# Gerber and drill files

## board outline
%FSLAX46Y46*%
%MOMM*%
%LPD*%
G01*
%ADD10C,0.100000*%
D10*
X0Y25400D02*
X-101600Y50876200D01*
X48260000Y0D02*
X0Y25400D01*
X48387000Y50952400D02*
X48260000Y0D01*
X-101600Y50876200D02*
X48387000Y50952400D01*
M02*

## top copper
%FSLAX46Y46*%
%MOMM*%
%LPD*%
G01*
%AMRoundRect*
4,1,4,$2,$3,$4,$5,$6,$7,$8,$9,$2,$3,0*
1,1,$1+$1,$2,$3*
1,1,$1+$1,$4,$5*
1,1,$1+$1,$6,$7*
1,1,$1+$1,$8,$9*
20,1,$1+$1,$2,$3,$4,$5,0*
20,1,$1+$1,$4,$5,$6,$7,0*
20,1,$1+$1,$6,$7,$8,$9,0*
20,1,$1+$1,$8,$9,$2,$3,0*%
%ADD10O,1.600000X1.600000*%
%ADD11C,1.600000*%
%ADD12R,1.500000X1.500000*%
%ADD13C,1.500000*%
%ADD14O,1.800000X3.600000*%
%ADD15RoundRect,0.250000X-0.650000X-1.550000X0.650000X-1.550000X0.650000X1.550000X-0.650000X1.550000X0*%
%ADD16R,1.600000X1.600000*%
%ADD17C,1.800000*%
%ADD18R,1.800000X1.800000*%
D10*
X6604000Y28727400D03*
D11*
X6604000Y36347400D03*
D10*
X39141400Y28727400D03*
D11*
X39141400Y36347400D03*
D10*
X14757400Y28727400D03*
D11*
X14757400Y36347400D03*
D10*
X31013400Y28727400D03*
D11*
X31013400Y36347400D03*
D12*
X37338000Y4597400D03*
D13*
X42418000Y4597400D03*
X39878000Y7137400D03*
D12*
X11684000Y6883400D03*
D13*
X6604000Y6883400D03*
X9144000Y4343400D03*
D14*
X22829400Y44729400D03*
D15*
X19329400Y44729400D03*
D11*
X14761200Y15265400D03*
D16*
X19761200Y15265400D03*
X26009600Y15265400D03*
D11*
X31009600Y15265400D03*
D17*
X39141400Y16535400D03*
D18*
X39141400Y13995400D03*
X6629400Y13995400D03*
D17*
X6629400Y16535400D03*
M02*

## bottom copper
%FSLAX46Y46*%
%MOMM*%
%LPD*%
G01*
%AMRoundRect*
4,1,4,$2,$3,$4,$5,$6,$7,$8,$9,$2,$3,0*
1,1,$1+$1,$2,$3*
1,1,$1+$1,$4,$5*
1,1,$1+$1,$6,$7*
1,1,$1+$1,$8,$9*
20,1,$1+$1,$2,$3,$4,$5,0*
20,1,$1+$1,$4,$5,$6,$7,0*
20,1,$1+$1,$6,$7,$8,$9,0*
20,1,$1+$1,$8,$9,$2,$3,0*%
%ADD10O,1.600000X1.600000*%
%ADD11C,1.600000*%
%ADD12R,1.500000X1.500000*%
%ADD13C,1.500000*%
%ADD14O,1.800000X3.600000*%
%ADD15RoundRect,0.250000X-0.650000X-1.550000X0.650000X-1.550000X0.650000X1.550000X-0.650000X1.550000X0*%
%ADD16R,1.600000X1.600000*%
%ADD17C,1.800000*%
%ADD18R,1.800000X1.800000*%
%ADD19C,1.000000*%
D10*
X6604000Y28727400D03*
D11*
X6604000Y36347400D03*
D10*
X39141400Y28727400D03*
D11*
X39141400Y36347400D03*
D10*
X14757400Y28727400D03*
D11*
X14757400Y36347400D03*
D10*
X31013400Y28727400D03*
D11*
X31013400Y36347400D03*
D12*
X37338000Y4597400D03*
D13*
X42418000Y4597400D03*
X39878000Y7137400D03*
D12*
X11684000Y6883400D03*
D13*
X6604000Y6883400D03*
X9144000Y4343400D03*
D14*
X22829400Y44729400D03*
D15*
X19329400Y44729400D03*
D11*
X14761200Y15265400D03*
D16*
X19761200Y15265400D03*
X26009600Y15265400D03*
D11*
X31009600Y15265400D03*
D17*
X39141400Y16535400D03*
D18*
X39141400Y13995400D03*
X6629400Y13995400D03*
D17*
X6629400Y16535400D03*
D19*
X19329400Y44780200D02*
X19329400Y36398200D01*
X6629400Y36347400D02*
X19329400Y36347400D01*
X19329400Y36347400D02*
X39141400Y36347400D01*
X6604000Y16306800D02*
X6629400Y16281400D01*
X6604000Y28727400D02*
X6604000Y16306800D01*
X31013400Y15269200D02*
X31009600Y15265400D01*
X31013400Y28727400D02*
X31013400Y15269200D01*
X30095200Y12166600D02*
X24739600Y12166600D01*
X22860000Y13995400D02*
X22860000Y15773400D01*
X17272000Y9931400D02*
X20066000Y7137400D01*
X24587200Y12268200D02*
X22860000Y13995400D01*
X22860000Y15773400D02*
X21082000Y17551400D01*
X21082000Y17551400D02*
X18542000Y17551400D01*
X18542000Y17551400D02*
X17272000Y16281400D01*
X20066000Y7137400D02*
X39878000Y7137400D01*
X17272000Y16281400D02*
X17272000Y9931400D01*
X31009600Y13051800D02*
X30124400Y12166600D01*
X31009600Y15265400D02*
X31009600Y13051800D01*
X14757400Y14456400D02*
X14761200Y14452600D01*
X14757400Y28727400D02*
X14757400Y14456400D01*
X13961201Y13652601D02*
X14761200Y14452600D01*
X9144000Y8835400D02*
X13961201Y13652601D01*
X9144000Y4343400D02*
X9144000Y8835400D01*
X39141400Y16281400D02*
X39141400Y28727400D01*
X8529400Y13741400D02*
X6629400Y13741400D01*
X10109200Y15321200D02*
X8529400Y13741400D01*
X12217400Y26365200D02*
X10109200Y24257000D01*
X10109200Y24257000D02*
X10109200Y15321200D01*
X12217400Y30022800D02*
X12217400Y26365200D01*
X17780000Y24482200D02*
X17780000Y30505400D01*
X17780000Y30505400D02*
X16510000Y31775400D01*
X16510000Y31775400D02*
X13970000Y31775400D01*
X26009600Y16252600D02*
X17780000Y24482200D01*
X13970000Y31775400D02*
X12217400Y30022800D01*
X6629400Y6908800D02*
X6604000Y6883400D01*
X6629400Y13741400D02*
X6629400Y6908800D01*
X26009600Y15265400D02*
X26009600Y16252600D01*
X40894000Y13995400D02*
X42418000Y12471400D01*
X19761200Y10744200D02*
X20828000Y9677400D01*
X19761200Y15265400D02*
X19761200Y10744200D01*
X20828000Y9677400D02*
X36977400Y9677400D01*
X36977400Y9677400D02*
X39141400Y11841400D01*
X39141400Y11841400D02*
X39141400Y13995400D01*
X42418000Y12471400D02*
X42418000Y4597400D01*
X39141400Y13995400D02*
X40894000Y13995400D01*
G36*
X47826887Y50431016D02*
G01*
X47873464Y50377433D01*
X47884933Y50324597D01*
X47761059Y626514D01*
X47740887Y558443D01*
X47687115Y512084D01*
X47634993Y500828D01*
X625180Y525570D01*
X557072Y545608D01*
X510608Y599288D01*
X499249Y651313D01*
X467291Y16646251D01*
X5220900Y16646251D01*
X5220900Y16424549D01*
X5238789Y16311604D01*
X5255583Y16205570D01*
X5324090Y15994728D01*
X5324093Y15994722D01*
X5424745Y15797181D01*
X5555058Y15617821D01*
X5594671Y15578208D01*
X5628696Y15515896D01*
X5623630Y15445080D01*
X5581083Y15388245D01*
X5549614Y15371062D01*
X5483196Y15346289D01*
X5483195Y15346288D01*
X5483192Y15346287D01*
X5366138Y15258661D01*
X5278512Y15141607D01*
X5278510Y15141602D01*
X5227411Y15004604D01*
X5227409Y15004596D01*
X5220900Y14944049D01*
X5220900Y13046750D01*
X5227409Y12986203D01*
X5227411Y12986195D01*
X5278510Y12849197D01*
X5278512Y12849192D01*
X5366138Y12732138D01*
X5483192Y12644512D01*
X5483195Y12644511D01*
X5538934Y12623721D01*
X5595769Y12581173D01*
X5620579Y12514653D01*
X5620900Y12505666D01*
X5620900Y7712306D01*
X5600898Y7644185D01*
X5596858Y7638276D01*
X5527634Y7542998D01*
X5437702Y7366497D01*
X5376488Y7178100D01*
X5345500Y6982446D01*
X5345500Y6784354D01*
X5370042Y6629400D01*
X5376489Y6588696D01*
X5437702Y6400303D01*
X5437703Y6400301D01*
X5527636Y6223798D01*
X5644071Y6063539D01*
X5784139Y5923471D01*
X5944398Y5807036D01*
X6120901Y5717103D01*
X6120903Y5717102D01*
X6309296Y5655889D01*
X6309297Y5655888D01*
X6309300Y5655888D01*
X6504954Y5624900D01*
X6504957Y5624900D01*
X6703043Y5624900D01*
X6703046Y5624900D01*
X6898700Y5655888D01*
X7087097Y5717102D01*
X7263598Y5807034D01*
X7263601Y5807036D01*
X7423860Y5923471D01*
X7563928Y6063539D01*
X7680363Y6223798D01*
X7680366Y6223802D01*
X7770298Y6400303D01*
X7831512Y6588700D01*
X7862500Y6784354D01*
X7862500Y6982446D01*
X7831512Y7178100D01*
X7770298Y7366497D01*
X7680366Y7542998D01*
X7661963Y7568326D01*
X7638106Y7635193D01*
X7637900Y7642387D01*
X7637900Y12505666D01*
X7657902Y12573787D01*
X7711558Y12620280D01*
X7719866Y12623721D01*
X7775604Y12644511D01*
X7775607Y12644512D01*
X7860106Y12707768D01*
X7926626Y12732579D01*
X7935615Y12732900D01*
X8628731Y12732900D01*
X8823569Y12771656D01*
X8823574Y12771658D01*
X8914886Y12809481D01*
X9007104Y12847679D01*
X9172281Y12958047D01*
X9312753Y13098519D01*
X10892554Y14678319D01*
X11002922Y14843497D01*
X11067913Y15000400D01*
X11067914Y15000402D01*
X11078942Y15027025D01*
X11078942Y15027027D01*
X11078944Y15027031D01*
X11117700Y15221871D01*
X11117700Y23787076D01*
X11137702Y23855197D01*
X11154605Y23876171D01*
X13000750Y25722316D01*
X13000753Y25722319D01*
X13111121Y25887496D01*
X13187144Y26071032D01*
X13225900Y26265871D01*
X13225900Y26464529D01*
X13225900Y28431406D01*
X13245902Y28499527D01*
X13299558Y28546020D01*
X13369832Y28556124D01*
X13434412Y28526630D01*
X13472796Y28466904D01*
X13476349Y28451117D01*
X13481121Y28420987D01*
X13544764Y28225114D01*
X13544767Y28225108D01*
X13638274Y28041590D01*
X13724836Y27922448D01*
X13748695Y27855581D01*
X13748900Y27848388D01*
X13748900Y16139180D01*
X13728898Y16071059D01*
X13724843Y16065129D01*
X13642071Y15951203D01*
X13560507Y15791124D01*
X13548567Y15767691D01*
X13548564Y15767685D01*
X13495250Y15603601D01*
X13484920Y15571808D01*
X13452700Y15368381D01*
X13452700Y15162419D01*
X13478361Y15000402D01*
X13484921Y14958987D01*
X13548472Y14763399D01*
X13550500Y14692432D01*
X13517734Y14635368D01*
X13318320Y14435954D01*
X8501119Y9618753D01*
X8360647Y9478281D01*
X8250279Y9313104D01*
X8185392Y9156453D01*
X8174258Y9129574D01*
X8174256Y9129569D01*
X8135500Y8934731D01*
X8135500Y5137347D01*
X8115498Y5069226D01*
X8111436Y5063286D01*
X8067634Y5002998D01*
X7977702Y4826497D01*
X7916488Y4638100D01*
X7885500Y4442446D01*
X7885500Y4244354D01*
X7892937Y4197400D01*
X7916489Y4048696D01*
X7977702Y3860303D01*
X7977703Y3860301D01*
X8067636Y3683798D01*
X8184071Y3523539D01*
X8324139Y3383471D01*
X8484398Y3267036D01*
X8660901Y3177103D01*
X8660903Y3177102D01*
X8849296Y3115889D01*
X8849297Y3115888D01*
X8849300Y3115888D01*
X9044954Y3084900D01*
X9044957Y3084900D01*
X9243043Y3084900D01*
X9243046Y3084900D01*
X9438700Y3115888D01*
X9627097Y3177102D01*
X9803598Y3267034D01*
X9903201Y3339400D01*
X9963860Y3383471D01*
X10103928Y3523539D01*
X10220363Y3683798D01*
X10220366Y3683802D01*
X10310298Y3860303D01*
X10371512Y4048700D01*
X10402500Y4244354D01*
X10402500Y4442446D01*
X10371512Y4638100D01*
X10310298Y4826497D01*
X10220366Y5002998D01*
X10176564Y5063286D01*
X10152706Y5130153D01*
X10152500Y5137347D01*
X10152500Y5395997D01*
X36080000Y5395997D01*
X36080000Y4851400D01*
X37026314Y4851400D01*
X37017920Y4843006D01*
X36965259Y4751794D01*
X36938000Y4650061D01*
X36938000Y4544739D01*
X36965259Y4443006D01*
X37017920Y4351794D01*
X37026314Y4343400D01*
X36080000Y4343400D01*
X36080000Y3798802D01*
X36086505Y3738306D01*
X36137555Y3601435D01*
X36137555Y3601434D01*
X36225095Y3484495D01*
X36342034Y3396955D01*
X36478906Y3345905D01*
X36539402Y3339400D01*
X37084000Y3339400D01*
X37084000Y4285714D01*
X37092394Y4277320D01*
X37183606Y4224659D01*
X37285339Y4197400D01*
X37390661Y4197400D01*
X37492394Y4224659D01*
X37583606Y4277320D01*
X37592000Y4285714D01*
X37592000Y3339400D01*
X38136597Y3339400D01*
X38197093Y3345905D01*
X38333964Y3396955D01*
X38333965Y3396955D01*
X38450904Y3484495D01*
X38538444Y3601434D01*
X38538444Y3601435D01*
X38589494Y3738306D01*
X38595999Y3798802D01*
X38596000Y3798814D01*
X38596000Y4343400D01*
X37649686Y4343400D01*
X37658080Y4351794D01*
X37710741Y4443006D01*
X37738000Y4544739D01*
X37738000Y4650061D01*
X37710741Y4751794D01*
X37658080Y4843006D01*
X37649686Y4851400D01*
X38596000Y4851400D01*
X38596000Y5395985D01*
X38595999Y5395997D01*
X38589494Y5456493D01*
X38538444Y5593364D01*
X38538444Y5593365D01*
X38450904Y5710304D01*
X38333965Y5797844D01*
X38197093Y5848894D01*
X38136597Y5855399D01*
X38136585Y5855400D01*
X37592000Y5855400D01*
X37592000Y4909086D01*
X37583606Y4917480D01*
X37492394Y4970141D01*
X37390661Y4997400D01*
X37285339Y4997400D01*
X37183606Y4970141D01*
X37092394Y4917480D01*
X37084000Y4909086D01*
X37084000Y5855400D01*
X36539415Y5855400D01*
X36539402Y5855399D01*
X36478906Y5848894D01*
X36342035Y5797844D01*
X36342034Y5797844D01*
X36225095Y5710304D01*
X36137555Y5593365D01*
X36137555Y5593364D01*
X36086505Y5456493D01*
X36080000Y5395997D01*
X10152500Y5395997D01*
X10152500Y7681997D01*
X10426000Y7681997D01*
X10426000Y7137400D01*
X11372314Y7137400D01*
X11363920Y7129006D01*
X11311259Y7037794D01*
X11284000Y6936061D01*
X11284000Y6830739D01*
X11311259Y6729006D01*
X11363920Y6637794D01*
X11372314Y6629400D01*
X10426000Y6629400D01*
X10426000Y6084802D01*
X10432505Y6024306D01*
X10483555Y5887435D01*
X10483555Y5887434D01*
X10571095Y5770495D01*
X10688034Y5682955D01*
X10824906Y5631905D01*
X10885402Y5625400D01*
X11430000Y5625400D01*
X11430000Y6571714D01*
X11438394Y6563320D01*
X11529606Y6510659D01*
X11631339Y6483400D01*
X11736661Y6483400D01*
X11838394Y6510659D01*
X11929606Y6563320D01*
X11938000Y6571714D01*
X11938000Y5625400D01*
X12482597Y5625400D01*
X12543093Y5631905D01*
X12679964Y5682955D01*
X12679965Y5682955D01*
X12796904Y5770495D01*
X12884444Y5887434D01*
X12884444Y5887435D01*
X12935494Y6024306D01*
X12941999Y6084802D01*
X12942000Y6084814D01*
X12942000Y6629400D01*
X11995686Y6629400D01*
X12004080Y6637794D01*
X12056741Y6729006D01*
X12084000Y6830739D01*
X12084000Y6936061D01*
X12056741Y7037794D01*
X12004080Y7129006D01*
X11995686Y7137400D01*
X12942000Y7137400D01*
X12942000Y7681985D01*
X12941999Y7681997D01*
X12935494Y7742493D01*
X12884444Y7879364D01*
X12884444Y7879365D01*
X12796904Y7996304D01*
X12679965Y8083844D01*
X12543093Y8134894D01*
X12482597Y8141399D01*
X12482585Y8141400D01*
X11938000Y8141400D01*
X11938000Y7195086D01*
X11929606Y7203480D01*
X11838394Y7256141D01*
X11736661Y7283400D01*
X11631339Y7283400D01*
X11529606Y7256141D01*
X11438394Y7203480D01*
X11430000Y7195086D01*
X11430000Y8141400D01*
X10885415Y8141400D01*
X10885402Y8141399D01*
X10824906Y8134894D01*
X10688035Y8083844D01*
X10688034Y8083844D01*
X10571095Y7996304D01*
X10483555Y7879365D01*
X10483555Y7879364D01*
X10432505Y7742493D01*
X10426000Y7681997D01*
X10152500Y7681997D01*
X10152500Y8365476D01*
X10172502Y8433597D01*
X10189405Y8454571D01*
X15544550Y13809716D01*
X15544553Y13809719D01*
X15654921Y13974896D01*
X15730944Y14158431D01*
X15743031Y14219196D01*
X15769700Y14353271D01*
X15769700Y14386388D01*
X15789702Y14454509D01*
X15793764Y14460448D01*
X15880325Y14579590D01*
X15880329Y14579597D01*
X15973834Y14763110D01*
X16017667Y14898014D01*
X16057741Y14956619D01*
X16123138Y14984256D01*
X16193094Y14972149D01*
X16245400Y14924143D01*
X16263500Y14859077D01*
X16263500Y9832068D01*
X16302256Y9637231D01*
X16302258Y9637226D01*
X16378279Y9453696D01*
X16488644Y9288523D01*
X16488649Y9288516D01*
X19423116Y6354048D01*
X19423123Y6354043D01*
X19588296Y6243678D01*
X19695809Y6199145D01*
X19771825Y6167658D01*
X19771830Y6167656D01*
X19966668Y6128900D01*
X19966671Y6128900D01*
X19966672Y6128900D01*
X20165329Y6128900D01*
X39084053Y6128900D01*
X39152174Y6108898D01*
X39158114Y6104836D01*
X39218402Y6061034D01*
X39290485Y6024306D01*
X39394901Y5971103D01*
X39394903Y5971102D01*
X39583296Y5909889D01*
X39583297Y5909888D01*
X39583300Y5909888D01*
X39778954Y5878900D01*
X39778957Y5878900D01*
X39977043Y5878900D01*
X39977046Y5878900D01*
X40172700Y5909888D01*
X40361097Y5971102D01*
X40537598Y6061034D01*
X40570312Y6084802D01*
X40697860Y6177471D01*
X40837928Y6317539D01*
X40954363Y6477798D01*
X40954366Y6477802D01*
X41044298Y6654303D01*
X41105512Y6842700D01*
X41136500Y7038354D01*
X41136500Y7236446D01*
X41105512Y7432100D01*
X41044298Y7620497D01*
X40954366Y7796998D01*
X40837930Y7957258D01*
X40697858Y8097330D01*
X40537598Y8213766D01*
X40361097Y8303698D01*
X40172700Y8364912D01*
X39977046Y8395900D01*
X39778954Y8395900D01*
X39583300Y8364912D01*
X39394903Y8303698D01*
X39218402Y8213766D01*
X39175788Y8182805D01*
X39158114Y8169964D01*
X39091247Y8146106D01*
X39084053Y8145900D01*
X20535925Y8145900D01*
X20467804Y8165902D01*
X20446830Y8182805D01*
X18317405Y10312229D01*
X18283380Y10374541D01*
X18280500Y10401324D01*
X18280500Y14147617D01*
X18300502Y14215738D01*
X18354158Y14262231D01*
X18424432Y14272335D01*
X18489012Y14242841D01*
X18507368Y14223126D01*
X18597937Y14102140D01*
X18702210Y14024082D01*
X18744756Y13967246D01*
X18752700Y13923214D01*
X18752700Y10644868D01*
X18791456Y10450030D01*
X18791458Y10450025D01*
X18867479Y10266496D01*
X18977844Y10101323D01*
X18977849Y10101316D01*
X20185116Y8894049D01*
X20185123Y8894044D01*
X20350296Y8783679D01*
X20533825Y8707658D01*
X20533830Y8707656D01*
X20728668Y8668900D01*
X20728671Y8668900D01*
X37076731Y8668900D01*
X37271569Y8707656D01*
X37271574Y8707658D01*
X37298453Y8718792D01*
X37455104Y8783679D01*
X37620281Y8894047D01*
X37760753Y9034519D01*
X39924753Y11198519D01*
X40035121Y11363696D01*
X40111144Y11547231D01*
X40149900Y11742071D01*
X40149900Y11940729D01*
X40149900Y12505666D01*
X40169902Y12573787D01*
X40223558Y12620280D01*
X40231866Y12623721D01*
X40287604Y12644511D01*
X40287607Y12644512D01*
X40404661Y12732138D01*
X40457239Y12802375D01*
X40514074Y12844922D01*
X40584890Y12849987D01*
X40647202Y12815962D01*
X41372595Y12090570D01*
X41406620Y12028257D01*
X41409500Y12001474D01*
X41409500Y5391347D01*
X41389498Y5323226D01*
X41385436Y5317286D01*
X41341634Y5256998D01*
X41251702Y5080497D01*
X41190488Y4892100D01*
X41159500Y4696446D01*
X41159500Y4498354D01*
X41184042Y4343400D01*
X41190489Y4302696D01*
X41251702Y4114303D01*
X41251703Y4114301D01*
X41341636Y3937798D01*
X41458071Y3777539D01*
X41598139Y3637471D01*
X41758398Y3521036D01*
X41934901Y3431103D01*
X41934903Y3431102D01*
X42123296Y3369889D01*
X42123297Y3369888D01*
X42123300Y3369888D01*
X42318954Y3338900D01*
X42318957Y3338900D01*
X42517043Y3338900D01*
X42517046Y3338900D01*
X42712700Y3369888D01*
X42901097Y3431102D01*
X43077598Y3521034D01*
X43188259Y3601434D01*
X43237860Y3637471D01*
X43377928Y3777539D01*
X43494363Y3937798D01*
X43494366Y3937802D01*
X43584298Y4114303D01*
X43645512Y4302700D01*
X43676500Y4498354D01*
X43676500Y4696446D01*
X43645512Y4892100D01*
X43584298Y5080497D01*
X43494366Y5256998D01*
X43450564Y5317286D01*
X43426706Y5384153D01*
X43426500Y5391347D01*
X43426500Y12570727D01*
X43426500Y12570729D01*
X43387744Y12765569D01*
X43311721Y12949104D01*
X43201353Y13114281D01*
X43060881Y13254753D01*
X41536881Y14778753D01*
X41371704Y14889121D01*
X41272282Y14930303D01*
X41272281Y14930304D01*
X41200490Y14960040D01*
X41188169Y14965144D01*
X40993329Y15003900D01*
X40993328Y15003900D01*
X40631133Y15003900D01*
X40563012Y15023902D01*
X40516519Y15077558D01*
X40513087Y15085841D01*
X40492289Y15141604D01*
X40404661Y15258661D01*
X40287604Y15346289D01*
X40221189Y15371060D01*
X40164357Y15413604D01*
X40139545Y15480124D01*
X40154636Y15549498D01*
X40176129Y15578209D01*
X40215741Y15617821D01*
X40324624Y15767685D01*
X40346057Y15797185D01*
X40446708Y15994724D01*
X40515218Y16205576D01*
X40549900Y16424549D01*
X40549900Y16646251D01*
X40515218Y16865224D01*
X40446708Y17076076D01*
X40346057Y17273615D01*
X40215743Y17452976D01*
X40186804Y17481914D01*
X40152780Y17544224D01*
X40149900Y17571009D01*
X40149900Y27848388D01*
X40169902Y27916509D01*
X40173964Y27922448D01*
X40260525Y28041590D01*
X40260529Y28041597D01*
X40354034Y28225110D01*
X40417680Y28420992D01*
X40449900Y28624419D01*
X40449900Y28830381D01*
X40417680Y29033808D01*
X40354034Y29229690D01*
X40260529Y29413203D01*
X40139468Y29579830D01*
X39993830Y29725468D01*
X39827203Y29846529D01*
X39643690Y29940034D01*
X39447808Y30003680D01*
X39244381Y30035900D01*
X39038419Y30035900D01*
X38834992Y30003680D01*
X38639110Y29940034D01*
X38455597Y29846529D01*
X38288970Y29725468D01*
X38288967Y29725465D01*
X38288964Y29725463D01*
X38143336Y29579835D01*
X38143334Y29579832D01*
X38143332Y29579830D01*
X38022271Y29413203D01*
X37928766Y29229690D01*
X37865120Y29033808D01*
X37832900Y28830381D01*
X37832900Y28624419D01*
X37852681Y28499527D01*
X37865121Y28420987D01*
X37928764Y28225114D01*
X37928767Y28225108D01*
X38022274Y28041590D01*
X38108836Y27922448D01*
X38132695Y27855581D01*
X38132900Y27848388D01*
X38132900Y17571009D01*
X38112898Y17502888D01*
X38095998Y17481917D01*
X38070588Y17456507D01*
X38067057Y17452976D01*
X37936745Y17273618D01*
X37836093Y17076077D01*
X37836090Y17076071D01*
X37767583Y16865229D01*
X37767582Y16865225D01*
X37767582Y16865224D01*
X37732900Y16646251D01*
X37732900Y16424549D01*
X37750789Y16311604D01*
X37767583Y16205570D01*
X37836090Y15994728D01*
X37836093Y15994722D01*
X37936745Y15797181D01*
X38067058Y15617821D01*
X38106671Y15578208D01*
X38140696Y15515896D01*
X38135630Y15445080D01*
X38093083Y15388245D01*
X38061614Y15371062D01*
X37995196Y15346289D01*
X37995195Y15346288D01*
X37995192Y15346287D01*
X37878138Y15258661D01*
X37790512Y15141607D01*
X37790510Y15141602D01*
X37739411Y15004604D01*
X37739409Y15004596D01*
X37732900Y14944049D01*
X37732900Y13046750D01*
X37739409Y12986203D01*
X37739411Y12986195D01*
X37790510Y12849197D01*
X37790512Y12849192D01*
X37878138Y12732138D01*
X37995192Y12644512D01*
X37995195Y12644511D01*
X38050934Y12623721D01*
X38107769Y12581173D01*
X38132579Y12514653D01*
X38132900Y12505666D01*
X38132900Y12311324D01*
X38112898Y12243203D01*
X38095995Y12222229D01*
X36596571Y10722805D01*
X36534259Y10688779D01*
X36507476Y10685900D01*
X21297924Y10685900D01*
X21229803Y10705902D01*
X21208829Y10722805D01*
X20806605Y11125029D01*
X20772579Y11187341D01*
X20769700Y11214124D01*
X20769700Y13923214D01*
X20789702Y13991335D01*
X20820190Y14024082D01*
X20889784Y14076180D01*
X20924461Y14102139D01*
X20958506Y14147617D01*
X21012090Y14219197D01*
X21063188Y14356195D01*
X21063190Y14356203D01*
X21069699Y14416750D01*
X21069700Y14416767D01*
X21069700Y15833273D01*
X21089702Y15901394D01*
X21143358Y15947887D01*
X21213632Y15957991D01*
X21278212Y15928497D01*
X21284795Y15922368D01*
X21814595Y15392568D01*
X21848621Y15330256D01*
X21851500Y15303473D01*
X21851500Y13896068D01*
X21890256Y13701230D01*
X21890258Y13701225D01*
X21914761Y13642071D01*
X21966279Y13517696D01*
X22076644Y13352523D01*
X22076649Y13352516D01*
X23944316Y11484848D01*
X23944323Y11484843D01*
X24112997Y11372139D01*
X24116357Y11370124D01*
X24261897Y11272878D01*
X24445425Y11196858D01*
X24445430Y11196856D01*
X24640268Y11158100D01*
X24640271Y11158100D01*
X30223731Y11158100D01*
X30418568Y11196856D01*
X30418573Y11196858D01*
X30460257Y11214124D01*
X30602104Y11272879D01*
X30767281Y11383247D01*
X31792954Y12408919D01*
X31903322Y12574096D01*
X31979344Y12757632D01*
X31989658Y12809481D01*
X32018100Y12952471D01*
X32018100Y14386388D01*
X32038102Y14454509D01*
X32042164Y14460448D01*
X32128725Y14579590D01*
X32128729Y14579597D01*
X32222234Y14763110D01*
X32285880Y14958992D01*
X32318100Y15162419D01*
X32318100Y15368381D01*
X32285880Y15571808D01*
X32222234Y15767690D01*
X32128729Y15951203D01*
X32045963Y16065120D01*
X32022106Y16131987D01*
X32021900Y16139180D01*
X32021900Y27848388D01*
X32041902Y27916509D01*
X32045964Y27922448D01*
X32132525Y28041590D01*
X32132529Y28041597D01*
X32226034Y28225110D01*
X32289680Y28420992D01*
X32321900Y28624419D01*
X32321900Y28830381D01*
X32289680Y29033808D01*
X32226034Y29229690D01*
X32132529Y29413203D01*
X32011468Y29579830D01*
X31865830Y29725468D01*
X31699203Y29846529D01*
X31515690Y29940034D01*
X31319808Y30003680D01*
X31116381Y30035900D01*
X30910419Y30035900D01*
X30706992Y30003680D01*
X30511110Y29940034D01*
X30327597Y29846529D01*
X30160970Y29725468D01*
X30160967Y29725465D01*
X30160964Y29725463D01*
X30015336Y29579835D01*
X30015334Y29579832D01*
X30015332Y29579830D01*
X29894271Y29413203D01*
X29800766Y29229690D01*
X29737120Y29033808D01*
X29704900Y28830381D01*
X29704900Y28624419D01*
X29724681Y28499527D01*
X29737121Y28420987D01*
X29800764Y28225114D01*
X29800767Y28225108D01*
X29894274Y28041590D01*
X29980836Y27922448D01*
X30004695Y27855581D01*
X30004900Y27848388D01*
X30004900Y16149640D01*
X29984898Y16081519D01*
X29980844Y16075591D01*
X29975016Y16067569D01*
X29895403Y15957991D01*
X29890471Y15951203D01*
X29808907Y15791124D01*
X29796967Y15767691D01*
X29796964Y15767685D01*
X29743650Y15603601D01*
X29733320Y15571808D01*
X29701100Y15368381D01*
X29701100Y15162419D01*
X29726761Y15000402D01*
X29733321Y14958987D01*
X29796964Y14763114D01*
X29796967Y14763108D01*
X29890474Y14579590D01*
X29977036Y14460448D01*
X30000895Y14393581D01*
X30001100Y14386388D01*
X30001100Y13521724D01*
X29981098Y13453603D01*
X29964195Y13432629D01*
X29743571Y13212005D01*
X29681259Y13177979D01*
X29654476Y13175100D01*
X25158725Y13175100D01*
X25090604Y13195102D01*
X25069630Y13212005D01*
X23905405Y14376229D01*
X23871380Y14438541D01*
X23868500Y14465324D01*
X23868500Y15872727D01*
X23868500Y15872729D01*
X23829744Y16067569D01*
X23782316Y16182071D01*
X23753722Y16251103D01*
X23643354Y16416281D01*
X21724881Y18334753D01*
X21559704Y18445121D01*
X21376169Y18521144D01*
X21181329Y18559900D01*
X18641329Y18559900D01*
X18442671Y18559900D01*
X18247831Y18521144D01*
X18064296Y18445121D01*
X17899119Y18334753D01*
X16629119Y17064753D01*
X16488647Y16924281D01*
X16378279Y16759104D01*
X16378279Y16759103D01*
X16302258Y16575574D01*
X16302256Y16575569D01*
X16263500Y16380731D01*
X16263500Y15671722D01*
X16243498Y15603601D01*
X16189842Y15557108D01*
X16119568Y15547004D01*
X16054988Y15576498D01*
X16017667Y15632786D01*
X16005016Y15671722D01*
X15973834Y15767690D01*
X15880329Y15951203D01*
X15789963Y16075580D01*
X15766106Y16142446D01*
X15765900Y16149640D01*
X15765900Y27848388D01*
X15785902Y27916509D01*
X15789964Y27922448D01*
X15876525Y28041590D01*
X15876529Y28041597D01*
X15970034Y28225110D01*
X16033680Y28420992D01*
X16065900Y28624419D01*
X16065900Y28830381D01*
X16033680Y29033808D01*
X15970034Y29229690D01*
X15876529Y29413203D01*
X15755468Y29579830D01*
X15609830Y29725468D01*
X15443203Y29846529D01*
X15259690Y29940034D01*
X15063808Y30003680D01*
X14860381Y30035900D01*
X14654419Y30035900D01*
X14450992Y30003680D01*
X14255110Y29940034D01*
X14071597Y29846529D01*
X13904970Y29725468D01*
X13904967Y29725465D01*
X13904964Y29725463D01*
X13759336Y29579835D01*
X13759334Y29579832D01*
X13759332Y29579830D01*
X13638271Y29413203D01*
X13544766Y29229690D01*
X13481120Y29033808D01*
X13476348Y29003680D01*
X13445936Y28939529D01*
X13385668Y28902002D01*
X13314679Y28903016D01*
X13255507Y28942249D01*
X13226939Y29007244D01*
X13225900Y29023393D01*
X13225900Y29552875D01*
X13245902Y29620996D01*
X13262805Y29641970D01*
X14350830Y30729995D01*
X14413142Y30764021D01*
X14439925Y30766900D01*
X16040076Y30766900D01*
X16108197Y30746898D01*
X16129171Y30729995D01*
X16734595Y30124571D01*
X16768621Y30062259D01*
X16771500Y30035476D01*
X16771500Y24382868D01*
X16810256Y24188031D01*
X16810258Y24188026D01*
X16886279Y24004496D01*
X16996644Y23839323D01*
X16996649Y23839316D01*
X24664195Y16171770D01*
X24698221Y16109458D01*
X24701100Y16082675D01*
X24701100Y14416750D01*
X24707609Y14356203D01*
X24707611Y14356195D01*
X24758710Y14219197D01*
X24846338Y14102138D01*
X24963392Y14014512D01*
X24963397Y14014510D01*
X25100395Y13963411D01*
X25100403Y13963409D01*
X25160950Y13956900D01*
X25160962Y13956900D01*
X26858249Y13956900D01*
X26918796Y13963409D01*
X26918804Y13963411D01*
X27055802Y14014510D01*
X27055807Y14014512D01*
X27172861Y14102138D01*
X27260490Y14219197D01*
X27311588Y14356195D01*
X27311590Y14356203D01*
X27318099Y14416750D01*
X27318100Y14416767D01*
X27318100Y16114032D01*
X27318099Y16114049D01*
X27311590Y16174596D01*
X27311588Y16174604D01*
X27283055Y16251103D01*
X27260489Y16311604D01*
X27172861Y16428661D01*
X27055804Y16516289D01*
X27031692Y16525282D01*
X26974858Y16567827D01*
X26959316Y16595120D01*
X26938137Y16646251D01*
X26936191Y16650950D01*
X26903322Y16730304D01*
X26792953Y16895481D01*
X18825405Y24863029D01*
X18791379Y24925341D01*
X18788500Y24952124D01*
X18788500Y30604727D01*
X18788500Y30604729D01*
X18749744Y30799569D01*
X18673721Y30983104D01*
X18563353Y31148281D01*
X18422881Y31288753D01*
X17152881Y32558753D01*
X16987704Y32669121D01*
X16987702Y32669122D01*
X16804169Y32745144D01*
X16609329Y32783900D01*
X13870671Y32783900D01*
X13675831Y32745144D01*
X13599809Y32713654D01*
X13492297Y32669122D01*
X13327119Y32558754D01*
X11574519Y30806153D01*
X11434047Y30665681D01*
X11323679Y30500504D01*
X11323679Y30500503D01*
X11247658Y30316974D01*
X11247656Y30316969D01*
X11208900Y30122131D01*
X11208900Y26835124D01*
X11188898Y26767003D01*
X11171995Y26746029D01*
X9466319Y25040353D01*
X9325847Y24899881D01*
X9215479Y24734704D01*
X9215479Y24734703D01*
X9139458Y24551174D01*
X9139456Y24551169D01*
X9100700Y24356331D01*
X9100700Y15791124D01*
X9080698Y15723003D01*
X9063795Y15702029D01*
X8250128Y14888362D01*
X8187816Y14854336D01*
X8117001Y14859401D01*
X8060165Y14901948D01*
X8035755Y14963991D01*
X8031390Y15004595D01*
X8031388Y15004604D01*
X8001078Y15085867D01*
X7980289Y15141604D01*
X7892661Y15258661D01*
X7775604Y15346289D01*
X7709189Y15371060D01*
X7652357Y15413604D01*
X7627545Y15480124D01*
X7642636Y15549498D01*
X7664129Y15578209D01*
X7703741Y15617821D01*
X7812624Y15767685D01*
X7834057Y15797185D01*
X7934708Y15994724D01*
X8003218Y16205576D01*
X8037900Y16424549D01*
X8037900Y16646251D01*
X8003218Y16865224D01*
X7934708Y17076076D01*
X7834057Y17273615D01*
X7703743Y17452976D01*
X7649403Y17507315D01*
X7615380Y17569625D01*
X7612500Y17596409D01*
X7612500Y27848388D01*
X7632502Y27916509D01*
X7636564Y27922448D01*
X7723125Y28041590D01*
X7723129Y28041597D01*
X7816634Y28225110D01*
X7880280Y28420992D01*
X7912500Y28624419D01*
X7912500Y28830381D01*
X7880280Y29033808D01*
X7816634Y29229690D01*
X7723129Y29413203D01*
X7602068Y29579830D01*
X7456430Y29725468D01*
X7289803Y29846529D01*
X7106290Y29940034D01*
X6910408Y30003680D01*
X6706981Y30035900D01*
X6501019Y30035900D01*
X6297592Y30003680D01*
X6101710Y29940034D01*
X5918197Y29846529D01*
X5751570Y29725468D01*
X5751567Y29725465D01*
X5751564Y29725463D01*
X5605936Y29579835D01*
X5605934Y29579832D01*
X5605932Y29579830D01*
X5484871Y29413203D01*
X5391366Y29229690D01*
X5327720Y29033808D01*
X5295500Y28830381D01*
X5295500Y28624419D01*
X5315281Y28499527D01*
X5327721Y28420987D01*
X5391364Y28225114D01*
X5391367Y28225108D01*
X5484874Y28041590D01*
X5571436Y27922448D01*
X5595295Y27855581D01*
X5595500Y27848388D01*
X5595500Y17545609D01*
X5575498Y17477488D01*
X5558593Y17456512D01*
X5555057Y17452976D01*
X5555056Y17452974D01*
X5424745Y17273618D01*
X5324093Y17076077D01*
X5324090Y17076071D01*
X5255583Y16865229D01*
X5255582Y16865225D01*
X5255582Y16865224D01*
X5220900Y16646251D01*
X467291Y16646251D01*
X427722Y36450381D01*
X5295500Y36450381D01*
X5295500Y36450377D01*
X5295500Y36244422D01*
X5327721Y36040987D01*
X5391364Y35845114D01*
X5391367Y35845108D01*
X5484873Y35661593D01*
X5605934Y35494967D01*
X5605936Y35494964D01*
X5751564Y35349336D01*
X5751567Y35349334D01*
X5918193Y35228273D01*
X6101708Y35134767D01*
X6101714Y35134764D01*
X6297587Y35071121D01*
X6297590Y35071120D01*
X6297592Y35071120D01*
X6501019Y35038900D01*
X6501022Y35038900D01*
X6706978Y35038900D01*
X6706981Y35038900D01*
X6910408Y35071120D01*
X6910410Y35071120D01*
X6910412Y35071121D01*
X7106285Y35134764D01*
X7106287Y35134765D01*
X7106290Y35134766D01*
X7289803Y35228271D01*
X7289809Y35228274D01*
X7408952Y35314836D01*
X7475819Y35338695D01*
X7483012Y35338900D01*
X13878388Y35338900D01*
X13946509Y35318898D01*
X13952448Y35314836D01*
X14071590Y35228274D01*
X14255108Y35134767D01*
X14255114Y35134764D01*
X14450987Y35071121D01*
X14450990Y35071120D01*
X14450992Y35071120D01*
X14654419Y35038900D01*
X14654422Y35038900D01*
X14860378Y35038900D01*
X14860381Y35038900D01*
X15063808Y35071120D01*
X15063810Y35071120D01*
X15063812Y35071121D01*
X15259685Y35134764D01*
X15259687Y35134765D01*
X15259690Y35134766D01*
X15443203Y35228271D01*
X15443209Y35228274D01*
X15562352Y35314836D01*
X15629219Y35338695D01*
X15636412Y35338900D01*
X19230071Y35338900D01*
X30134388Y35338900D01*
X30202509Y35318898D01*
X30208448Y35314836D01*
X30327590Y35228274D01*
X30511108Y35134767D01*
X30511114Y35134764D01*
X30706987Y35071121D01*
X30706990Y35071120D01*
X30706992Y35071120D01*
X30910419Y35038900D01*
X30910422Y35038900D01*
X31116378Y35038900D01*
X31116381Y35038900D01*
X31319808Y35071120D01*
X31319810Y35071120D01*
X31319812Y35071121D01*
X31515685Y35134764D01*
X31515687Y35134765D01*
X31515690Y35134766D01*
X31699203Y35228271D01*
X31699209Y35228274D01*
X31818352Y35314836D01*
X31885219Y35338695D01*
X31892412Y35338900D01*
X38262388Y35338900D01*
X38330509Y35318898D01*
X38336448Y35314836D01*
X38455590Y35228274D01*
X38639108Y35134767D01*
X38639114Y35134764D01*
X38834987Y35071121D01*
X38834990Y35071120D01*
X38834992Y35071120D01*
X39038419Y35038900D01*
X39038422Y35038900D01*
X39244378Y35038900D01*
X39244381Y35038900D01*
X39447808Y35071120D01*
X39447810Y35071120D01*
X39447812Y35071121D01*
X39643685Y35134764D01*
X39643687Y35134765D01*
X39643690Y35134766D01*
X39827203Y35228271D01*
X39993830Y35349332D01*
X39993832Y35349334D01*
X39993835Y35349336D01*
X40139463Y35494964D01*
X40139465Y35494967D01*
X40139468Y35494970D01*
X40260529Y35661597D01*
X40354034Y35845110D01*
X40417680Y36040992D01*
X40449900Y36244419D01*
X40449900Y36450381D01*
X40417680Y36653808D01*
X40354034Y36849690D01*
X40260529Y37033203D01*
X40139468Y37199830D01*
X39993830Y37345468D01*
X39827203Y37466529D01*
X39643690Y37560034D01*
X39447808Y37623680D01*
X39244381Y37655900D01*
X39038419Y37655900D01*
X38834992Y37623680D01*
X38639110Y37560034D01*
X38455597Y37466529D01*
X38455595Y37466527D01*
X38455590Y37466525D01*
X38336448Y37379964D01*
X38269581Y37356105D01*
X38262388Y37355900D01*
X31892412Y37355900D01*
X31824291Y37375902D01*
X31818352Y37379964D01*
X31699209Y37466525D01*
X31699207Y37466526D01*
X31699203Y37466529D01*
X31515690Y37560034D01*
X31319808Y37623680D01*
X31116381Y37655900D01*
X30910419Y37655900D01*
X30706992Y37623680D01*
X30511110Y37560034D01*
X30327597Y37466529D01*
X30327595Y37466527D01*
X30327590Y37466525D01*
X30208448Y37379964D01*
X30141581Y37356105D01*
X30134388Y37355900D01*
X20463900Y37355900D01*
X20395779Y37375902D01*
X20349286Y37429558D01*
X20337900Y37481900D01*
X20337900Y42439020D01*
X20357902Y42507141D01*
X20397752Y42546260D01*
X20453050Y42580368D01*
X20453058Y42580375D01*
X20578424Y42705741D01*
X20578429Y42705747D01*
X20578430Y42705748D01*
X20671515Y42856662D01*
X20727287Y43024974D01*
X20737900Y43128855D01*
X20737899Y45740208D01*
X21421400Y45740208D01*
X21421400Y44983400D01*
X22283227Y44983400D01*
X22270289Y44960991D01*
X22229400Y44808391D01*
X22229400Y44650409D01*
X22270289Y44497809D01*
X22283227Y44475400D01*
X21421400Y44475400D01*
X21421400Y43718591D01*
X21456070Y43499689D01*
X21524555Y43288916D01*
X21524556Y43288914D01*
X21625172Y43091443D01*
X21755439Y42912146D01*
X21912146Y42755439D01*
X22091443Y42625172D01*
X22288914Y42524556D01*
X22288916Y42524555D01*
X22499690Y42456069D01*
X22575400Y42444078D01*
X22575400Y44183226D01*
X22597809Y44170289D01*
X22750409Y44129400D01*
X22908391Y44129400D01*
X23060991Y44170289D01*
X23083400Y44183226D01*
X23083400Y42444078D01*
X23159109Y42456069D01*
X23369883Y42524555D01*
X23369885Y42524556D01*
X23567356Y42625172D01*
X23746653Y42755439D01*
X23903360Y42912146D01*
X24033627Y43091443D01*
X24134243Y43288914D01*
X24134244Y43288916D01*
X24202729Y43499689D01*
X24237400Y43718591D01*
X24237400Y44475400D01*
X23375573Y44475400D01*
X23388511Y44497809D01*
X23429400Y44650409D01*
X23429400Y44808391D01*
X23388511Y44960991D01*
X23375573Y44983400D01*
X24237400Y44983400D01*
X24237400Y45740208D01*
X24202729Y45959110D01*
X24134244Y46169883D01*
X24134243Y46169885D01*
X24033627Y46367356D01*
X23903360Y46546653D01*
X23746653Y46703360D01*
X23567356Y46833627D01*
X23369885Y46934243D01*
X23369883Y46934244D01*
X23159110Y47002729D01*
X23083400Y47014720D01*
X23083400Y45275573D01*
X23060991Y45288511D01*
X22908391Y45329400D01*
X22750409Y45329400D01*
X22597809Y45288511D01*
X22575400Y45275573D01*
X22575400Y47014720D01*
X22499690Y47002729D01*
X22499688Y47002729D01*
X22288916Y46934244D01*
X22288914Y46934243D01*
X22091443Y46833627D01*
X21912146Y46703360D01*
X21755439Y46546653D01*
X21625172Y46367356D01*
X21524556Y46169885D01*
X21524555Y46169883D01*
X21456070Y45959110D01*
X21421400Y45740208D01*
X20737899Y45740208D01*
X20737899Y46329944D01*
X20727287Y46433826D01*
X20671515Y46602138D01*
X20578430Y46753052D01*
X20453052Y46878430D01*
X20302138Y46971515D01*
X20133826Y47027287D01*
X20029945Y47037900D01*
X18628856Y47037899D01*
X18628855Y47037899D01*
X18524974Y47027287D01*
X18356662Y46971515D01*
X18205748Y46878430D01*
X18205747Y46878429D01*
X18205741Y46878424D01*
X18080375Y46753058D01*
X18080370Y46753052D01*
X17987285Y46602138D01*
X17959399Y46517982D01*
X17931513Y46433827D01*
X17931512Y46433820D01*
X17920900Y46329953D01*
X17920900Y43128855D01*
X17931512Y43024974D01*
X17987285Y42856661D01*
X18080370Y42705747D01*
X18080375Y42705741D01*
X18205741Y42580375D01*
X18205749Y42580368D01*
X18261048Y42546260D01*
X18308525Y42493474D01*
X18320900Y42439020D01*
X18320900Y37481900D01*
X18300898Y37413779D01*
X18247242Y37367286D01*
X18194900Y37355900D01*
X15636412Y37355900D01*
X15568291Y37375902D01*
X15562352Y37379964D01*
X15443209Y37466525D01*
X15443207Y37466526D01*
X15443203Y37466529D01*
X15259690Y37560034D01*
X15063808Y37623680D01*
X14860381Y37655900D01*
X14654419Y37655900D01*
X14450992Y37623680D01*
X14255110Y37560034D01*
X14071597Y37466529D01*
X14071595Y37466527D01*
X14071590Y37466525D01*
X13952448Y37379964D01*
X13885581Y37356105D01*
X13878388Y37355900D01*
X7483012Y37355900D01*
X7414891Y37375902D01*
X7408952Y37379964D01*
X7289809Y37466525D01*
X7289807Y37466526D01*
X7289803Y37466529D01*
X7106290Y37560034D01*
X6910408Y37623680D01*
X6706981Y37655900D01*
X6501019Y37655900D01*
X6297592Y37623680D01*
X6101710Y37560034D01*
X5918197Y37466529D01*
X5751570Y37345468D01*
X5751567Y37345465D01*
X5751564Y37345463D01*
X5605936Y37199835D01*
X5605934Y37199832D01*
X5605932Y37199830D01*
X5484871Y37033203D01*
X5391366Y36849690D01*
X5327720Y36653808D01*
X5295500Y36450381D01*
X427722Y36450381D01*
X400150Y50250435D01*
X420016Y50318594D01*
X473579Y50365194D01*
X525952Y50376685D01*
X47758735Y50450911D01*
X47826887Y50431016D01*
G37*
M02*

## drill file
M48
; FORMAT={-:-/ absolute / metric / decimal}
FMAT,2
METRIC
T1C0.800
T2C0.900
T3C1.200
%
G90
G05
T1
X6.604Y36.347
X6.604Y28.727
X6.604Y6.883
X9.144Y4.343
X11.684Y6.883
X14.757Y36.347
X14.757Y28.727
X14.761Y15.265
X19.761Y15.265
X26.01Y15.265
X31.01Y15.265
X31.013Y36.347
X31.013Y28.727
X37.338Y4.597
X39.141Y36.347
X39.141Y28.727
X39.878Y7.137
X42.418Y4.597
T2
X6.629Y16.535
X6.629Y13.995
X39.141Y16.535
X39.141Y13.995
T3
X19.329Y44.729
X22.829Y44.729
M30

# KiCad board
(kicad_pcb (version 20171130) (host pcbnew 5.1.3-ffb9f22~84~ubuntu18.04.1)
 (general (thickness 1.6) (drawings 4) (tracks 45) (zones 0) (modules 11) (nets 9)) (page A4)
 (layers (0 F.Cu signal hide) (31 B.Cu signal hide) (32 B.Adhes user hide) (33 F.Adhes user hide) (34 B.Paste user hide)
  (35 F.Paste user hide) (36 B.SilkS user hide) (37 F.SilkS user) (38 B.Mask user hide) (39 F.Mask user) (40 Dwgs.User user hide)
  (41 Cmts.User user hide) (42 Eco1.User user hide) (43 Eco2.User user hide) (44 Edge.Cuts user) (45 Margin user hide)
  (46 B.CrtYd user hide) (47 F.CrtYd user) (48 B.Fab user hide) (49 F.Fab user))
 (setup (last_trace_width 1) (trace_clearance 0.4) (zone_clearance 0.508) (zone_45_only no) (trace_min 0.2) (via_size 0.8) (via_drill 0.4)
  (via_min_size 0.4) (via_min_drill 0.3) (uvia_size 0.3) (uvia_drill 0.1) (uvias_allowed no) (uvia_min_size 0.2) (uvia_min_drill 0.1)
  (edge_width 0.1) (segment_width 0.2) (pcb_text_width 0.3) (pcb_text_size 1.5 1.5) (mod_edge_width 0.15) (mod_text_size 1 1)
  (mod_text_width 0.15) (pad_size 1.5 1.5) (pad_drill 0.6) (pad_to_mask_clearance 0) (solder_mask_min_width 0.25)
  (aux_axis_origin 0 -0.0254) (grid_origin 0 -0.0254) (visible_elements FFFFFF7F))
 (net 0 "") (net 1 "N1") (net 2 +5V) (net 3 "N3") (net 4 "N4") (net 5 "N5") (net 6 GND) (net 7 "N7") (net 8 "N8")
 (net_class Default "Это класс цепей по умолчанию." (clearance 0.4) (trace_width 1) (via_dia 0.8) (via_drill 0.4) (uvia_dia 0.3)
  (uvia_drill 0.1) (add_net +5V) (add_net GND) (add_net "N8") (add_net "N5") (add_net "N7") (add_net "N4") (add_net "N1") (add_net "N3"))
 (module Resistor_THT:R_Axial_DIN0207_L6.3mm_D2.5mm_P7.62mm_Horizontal (layer F.Cu) (at 6.604 -36.3474 270)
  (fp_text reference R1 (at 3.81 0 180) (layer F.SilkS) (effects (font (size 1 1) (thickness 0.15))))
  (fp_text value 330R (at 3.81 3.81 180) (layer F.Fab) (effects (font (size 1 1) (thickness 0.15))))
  (pad 2 thru_hole oval (at 7.62 0 270) (size 1.6 1.6) (drill 0.8) (layers *.Cu *.Mask) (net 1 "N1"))
  (pad 1 thru_hole circle (at 0 0 270) (size 1.6 1.6) (drill 0.8) (layers *.Cu *.Mask) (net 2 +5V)))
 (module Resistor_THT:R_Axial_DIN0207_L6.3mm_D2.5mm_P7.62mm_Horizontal (layer F.Cu) (at 39.1414 -36.3474 270)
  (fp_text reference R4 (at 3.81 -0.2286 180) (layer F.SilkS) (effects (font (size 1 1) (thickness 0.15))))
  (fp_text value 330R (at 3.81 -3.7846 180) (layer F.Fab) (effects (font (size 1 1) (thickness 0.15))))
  (pad 2 thru_hole oval (at 7.62 0 270) (size 1.6 1.6) (drill 0.8) (layers *.Cu *.Mask) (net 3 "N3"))
  (pad 1 thru_hole circle (at 0 0 270) (size 1.6 1.6) (drill 0.8) (layers *.Cu *.Mask) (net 2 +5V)))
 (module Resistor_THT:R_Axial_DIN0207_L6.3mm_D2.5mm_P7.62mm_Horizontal (layer F.Cu) (at 14.7574 -36.3474 270)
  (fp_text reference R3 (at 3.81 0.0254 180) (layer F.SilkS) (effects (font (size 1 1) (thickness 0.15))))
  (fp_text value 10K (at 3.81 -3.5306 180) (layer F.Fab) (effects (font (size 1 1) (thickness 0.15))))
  (pad 2 thru_hole oval (at 7.62 0 270) (size 1.6 1.6) (drill 0.8) (layers *.Cu *.Mask) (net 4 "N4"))
  (pad 1 thru_hole circle (at 0 0 270) (size 1.6 1.6) (drill 0.8) (layers *.Cu *.Mask) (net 2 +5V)))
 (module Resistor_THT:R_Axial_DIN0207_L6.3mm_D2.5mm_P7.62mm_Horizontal (layer F.Cu) (at 31.0134 -36.3474 270)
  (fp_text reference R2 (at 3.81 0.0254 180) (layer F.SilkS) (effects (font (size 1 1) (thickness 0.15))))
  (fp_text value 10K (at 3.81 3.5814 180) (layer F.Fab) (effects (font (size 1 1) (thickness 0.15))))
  (pad 2 thru_hole oval (at 7.62 0 270) (size 1.6 1.6) (drill 0.8) (layers *.Cu *.Mask) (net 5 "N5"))
  (pad 1 thru_hole circle (at 0 0 270) (size 1.6 1.6) (drill 0.8) (layers *.Cu *.Mask) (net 2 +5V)))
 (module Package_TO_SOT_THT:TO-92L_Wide (layer F.Cu) (at 37.338 -4.5974)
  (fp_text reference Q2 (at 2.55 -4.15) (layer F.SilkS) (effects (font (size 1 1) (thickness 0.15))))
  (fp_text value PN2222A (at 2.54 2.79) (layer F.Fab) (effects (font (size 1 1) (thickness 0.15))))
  (pad 1 thru_hole rect (at 0 0 90) (size 1.5 1.5) (drill 0.8) (layers *.Cu *.Mask) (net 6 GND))
  (pad 3 thru_hole circle (at 5.08 0 90) (size 1.5 1.5) (drill 0.8) (layers *.Cu *.Mask) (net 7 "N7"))
  (pad 2 thru_hole circle (at 2.54 -2.54 90) (size 1.5 1.5) (drill 0.8) (layers *.Cu *.Mask) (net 5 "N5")))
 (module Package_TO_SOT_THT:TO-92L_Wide (layer F.Cu) (at 11.684 -6.8834 180)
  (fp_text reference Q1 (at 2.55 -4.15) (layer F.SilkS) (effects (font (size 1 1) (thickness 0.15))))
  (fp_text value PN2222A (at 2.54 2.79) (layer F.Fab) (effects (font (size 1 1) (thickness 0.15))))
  (pad 1 thru_hole rect (at 0 0 270) (size 1.5 1.5) (drill 0.8) (layers *.Cu *.Mask) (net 6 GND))
  (pad 3 thru_hole circle (at 5.08 0 270) (size 1.5 1.5) (drill 0.8) (layers *.Cu *.Mask) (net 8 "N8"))
  (pad 2 thru_hole circle (at 2.54 -2.54 270) (size 1.5 1.5) (drill 0.8) (layers *.Cu *.Mask) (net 4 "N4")))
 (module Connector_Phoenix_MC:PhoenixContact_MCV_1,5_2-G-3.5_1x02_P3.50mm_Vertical (layer F.Cu) (at 19.3294 -44.7294)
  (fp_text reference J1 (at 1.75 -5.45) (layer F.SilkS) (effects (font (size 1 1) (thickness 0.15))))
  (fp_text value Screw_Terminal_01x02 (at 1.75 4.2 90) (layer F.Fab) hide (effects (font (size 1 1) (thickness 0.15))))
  (pad 2 thru_hole oval (at 3.5 0) (size 1.8 3.6) (drill 1.2) (layers *.Cu *.Mask) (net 6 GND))
  (pad 1 thru_hole roundrect (at 0 0) (size 1.8 3.6) (drill 1.2) (layers *.Cu *.Mask) (roundrect_rratio 0.138889) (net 2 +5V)))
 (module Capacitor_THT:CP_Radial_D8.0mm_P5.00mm (layer F.Cu) (at 19.7612 -15.2654 180)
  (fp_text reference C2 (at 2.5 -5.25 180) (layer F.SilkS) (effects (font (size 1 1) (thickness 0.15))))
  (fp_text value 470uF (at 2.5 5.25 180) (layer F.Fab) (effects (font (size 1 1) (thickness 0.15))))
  (pad 2 thru_hole circle (at 5 0 180) (size 1.6 1.6) (drill 0.8) (layers *.Cu *.Mask) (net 4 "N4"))
  (pad 1 thru_hole rect (at 0 0 180) (size 1.6 1.6) (drill 0.8) (layers *.Cu *.Mask) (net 7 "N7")))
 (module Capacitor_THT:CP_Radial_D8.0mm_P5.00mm (layer F.Cu) (at 26.0096 -15.2654)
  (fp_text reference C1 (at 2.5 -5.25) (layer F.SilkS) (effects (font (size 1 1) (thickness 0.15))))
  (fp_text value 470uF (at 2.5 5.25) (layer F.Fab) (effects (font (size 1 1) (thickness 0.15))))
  (pad 1 thru_hole rect (at 0 0) (size 1.6 1.6) (drill 0.8) (layers *.Cu *.Mask) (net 8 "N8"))
  (pad 2 thru_hole circle (at 5 0) (size 1.6 1.6) (drill 0.8) (layers *.Cu *.Mask) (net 5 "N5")))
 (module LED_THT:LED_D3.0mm (layer F.Cu) (at 39.1414 -13.9954 90)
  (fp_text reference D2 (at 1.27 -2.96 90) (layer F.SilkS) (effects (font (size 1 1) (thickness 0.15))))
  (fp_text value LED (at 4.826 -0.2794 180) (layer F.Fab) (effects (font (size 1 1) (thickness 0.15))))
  (pad 2 thru_hole circle (at 2.54 0 90) (size 1.8 1.8) (drill 0.9) (layers *.Cu *.Mask) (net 3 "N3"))
  (pad 1 thru_hole rect (at 0 0 90) (size 1.8 1.8) (drill 0.9) (layers *.Cu *.Mask) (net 7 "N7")))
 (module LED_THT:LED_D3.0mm (layer F.Cu) (at 6.6294 -13.9954 90)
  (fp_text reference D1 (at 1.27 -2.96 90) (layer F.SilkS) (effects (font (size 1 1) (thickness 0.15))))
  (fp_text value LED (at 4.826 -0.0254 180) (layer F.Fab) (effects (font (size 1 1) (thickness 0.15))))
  (pad 1 thru_hole rect (at 0 0 90) (size 1.8 1.8) (drill 0.9) (layers *.Cu *.Mask) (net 8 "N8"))
  (pad 2 thru_hole circle (at 2.54 0 90) (size 1.8 1.8) (drill 0.9) (layers *.Cu *.Mask) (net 1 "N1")))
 (gr_line (start 0 -0.0254) (end -0.1016 -50.8762) (layer Edge.Cuts) (width 0.1))
 (gr_line (start 48.26 0) (end 0 -0.0254) (layer Edge.Cuts) (width 0.1))
 (gr_line (start 48.387 -50.9524) (end 48.26 0) (layer Edge.Cuts) (width 0.1))
 (gr_line (start -0.1016 -50.8762) (end 48.387 -50.9524) (layer Edge.Cuts) (width 0.1))
 (segment (start 19.3294 -44.7802) (end 19.3294 -36.3982) (width 1) (layer B.Cu) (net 2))
 (segment (start 6.6294 -36.3474) (end 19.3294 -36.3474) (width 1) (layer B.Cu) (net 2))
 (segment (start 19.3294 -36.3474) (end 39.1414 -36.3474) (width 1) (layer B.Cu) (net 2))
 (segment (start 6.604 -16.3068) (end 6.6294 -16.2814) (width 1) (layer B.Cu) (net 1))
 (segment (start 6.604 -28.7274) (end 6.604 -16.3068) (width 1) (layer B.Cu) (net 1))
 (segment (start 31.0134 -15.2692) (end 31.0096 -15.2654) (width 1) (layer B.Cu) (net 5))
 (segment (start 31.0134 -28.7274) (end 31.0134 -15.2692) (width 1) (layer B.Cu) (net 5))
 (segment (start 30.0952 -12.1666) (end 24.7396 -12.1666) (width 1) (layer B.Cu) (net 5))
 (segment (start 22.86 -13.9954) (end 22.86 -15.7734) (width 1) (layer B.Cu) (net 5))
 (segment (start 17.272 -9.9314) (end 20.066 -7.1374) (width 1) (layer B.Cu) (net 5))
 (segment (start 24.5872 -12.2682) (end 22.86 -13.9954) (width 1) (layer B.Cu) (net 5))
 (segment (start 22.86 -15.7734) (end 21.082 -17.5514) (width 1) (layer B.Cu) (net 5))
 (segment (start 21.082 -17.5514) (end 18.542 -17.5514) (width 1) (layer B.Cu) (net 5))
 (segment (start 18.542 -17.5514) (end 17.272 -16.2814) (width 1) (layer B.Cu) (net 5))
 (segment (start 20.066 -7.1374) (end 39.878 -7.1374) (width 1) (layer B.Cu) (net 5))
 (segment (start 17.272 -16.2814) (end 17.272 -9.9314) (width 1) (layer B.Cu) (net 5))
 (segment (start 31.0096 -13.0518) (end 30.1244 -12.1666) (width 1) (layer B.Cu) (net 5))
 (segment (start 31.0096 -15.2654) (end 31.0096 -13.0518) (width 1) (layer B.Cu) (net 5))
 (segment (start 14.7574 -14.4564) (end 14.7612 -14.4526) (width 1) (layer B.Cu) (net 4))
 (segment (start 14.7574 -28.7274) (end 14.7574 -14.4564) (width 1) (layer B.Cu) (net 4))
 (segment (start 13.961201 -13.652601) (end 14.7612 -14.4526) (width 1) (layer B.Cu) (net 4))
 (segment (start 9.144 -8.8354) (end 13.961201 -13.652601) (width 1) (layer B.Cu) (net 4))
 (segment (start 9.144 -4.3434) (end 9.144 -8.8354) (width 1) (layer B.Cu) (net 4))
 (segment (start 39.1414 -16.2814) (end 39.1414 -28.7274) (width 1) (layer B.Cu) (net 3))
 (segment (start 8.5294 -13.7414) (end 6.6294 -13.7414) (width 1) (layer B.Cu) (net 8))
 (segment (start 10.1092 -15.3212) (end 8.5294 -13.7414) (width 1) (layer B.Cu) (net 8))
 (segment (start 12.2174 -26.3652) (end 10.1092 -24.257) (width 1) (layer B.Cu) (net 8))
 (segment (start 10.1092 -24.257) (end 10.1092 -15.3212) (width 1) (layer B.Cu) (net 8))
 (segment (start 12.2174 -30.0228) (end 12.2174 -26.3652) (width 1) (layer B.Cu) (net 8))
 (segment (start 17.78 -24.4822) (end 17.78 -30.5054) (width 1) (layer B.Cu) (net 8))
 (segment (start 17.78 -30.5054) (end 16.51 -31.7754) (width 1) (layer B.Cu) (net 8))
 (segment (start 16.51 -31.7754) (end 13.97 -31.7754) (width 1) (layer B.Cu) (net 8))
 (segment (start 26.0096 -16.2526) (end 17.78 -24.4822) (width 1) (layer B.Cu) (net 8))
 (segment (start 13.97 -31.7754) (end 12.2174 -30.0228) (width 1) (layer B.Cu) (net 8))
 (segment (start 6.6294 -6.9088) (end 6.604 -6.8834) (width 1) (layer B.Cu) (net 8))
 (segment (start 6.6294 -13.7414) (end 6.6294 -6.9088) (width 1) (layer B.Cu) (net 8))
 (segment (start 26.0096 -15.2654) (end 26.0096 -16.2526) (width 1) (layer B.Cu) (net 8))
 (segment (start 40.894 -13.9954) (end 42.418 -12.4714) (width 1) (layer B.Cu) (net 7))
 (segment (start 19.7612 -10.7442) (end 20.828 -9.6774) (width 1) (layer B.Cu) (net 7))
 (segment (start 19.7612 -15.2654) (end 19.7612 -10.7442) (width 1) (layer B.Cu) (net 7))
 (segment (start 20.828 -9.6774) (end 36.9774 -9.6774) (width 1) (layer B.Cu) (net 7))
 (segment (start 36.9774 -9.6774) (end 39.1414 -11.8414) (width 1) (layer B.Cu) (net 7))
 (segment (start 39.1414 -11.8414) (end 39.1414 -13.9954) (width 1) (layer B.Cu) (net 7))
 (segment (start 42.418 -12.4714) (end 42.418 -4.5974) (width 1) (layer B.Cu) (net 7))
 (segment (start 39.1414 -13.9954) (end 40.894 -13.9954) (width 1) (layer B.Cu) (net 7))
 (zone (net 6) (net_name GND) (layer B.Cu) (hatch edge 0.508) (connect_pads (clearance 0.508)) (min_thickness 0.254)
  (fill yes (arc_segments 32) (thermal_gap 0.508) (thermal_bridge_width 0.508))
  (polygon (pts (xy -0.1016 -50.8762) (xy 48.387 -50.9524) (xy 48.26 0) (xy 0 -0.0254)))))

